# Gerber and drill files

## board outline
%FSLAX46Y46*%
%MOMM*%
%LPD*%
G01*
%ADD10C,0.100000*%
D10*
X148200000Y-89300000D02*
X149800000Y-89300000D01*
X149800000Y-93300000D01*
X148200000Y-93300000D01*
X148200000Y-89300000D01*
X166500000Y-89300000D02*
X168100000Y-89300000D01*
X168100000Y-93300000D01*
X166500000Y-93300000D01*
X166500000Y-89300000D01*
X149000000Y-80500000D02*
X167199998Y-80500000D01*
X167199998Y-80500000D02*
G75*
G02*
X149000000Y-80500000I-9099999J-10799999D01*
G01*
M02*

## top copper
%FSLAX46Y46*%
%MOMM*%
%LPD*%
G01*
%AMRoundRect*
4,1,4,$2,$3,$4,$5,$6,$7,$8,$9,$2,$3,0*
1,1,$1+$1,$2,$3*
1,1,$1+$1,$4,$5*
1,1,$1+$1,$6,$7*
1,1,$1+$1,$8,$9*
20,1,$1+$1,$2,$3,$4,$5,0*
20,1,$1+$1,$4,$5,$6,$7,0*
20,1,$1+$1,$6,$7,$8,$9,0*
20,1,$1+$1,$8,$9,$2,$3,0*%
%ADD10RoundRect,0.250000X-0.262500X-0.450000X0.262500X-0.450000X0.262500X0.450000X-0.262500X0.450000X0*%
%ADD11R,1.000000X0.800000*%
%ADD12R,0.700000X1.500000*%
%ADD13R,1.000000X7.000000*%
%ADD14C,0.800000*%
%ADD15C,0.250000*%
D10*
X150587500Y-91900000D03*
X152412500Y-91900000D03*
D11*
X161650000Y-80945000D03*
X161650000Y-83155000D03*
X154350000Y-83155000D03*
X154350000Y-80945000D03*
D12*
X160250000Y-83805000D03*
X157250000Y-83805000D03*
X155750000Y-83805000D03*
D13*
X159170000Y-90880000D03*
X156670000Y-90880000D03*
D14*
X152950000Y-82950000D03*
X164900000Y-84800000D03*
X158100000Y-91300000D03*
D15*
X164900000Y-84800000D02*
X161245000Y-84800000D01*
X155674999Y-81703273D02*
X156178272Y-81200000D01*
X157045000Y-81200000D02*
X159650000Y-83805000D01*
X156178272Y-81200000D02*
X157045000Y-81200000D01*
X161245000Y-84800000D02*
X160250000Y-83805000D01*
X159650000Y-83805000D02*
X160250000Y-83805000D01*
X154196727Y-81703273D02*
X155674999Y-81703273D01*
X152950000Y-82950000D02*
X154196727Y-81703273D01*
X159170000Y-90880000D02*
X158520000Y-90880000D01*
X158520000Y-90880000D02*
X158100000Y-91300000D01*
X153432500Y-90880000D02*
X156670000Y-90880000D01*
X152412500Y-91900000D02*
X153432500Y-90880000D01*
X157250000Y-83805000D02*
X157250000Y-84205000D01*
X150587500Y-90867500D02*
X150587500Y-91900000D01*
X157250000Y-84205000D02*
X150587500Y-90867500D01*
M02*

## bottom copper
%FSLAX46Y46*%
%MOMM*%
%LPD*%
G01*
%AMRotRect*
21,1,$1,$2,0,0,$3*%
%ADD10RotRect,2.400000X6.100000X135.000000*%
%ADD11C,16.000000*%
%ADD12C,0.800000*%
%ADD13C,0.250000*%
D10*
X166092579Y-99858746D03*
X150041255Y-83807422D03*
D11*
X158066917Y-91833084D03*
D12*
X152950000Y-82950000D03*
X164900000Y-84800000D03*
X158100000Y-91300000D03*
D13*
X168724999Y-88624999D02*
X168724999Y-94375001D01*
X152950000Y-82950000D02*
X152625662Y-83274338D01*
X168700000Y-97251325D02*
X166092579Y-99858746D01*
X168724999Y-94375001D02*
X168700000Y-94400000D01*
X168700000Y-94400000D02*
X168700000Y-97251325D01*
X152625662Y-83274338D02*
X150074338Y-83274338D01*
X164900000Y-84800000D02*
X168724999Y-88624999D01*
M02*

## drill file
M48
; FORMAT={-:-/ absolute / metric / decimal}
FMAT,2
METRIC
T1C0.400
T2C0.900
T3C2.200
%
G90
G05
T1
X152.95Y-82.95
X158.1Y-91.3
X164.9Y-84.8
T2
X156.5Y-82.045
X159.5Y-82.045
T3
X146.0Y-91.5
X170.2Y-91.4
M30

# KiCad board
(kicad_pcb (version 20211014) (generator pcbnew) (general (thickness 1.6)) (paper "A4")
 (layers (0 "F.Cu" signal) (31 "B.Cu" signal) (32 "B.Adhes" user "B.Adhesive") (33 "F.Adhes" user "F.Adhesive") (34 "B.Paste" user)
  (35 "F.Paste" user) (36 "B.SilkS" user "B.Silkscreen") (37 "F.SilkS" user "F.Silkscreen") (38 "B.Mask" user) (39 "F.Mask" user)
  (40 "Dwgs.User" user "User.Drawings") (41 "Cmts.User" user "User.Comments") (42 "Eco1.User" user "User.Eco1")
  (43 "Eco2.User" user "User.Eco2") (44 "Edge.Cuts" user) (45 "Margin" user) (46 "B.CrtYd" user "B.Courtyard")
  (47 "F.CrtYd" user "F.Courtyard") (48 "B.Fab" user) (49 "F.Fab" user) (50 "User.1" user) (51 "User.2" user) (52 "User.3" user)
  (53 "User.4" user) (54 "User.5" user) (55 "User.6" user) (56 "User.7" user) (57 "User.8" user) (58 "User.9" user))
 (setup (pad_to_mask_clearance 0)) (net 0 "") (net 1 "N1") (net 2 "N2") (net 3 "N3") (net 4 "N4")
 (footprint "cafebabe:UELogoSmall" (layer "F.Cu") (at 158.6 97)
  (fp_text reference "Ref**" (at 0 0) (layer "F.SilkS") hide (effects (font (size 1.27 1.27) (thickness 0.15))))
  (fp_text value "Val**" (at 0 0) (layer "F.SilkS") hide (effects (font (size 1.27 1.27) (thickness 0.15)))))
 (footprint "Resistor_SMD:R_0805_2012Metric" (layer "F.Cu") (at 151.5 91.9)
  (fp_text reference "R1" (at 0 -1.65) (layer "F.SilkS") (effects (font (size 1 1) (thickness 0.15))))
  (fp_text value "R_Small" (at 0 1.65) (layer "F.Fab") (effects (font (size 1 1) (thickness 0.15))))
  (pad "1" smd roundrect (at -0.9125 0) (size 1.025 1.4) (layers "F.Cu" "F.Paste" "F.Mask") (roundrect_rratio 0.243902439) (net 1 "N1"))
  (pad "2" smd roundrect (at 0.9125 0) (size 1.025 1.4) (layers "F.Cu" "F.Paste" "F.Mask") (roundrect_rratio 0.243902439) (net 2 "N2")))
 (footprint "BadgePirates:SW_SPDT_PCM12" (layer "F.Cu") (at 158 82.375 180)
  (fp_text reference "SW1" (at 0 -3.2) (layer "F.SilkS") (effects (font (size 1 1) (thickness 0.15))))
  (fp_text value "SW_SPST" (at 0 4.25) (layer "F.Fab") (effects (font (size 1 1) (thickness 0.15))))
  (pad "" smd rect locked (at -3.65 1.43 180) (size 1 0.8) (layers "F.Cu" "F.Paste" "F.Mask"))
  (pad "" np_thru_hole circle locked (at -1.5 0.33 180) (size 0.9 0.9) (drill 0.9) (layers *.Cu *.Mask))
  (pad "" smd rect locked (at -3.65 -0.78 180) (size 1 0.8) (layers "F.Cu" "F.Paste" "F.Mask"))
  (pad "" smd rect locked (at 3.65 -0.78 180) (size 1 0.8) (layers "F.Cu" "F.Paste" "F.Mask"))
  (pad "" np_thru_hole circle locked (at 1.5 0.33 180) (size 0.9 0.9) (drill 0.9) (layers *.Cu *.Mask))
  (pad "" smd rect locked (at 3.65 1.43 180) (size 1 0.8) (layers "F.Cu" "F.Paste" "F.Mask"))
  (pad "1" smd rect locked (at -2.25 -1.43 180) (size 0.7 1.5) (layers "F.Cu" "F.Paste" "F.Mask") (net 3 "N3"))
  (pad "2" smd rect locked (at 0.75 -1.43 180) (size 0.7 1.5) (layers "F.Cu" "F.Paste" "F.Mask") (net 1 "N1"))
  (pad "3" smd rect locked (at 2.25 -1.43 180) (size 0.7 1.5) (layers "F.Cu" "F.Paste" "F.Mask")))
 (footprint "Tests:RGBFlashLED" (layer "F.Cu") (at 159.17 90.88 180)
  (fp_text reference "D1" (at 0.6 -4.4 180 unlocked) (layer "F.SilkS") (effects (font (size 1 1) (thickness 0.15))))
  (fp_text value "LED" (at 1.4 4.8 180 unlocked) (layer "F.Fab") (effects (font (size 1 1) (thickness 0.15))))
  (pad "1" smd rect (at 0 0 180) (size 1 7) (layers "F.Cu" "F.Paste" "F.Mask") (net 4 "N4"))
  (pad "2" smd rect (at 2.5 0 180) (size 1 7) (layers "F.Cu" "F.Paste" "F.Mask") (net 2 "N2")))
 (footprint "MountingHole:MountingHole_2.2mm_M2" (layer "F.Cu") (at 170.2 91.4)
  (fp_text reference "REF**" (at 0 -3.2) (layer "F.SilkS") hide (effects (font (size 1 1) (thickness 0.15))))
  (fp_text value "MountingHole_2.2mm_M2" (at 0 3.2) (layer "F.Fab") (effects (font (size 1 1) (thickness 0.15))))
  (pad "" np_thru_hole circle (at 0 0) (size 2.2 2.2) (drill 2.2) (layers *.Cu *.Mask)))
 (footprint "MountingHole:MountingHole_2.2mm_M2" (layer "F.Cu") (at 146 91.5)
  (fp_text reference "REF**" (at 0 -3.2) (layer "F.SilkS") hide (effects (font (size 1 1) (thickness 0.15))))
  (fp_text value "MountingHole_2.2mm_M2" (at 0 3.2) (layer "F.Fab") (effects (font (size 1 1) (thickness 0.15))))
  (pad "" np_thru_hole circle (at 0 0) (size 2.2 2.2) (drill 2.2) (layers *.Cu *.Mask)))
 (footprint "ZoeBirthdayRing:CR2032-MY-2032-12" (layer "B.Cu") (at 158.066917 91.833084 135)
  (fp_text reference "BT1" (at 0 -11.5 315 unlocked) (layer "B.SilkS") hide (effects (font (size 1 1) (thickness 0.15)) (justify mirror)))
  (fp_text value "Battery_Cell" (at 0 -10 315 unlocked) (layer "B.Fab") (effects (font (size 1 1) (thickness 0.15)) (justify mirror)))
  (pad "1" smd rect (at -11.35 0 135) (size 2.4 6.1) (layers "B.Cu" "B.Paste" "B.Mask") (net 3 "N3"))
  (pad "1" smd rect (at 11.35 0 135) (size 2.4 6.1) (layers "B.Cu" "B.Paste" "B.Mask") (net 3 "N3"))
  (pad "2" smd circle (at 0 0 135) (size 16 16) (layers "B.Cu" "B.Paste" "B.Mask") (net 4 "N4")))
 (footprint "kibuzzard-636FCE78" (layer "B.Cu") (at 158.1 102.1 180)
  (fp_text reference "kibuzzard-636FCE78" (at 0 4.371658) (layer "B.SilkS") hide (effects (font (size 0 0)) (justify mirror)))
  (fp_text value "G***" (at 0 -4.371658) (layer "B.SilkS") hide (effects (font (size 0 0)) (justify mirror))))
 (gr_rect (start 148.2 89.3) (end 149.8 93.3) (layer "Edge.Cuts") (width 0.1) (fill none))
 (gr_rect (start 166.5 89.3) (end 168.1 93.3) (layer "Edge.Cuts") (width 0.1) (fill none))
 (gr_line (start 149 80.5) (end 167.199998 80.5) (layer "Edge.Cuts") (width 0.1))
 (gr_arc (start 167.199998 80.5) (mid 158.099999 105.422674) (end 149 80.5) (layer "Edge.Cuts") (width 0.1))
 (segment (start 164.9 84.8) (end 161.245 84.8) (width 0.25) (layer "F.Cu") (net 3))
 (segment (start 155.674999 81.703273) (end 156.178272 81.2) (width 0.25) (layer "F.Cu") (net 3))
 (segment (start 157.045 81.2) (end 159.65 83.805) (width 0.25) (layer "F.Cu") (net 3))
 (segment (start 156.178272 81.2) (end 157.045 81.2) (width 0.25) (layer "F.Cu") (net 3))
 (segment (start 161.245 84.8) (end 160.25 83.805) (width 0.25) (layer "F.Cu") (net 3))
 (segment (start 159.65 83.805) (end 160.25 83.805) (width 0.25) (layer "F.Cu") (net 3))
 (segment (start 154.196727 81.703273) (end 155.674999 81.703273) (width 0.25) (layer "F.Cu") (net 3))
 (segment (start 152.95 82.95) (end 154.196727 81.703273) (width 0.25) (layer "F.Cu") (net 3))
 (via (at 152.95 82.95) (size 0.8) (drill 0.4) (layers "F.Cu" "B.Cu") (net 3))
 (via (at 164.9 84.8) (size 0.8) (drill 0.4) (layers "F.Cu" "B.Cu") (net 3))
 (segment (start 168.724999 88.624999) (end 168.724999 94.375001) (width 0.25) (layer "B.Cu") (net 3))
 (segment (start 152.95 82.95) (end 152.625662 83.274338) (width 0.25) (layer "B.Cu") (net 3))
 (segment (start 168.7 97.251325) (end 166.092579 99.858746) (width 0.25) (layer "B.Cu") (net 3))
 (segment (start 168.724999 94.375001) (end 168.7 94.4) (width 0.25) (layer "B.Cu") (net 3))
 (segment (start 168.7 94.4) (end 168.7 97.251325) (width 0.25) (layer "B.Cu") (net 3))
 (segment (start 152.625662 83.274338) (end 150.074338 83.274338) (width 0.25) (layer "B.Cu") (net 3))
 (segment (start 164.9 84.8) (end 168.724999 88.624999) (width 0.25) (layer "B.Cu") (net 3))
 (segment (start 159.17 90.88) (end 158.52 90.88) (width 0.25) (layer "F.Cu") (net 4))
 (segment (start 158.52 90.88) (end 158.1 91.3) (width 0.25) (layer "F.Cu") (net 4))
 (via (at 158.1 91.3) (size 0.8) (drill 0.4) (layers "F.Cu" "B.Cu") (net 4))
 (segment (start 153.4325 90.88) (end 156.67 90.88) (width 0.25) (layer "F.Cu") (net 2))
 (segment (start 152.4125 91.9) (end 153.4325 90.88) (width 0.25) (layer "F.Cu") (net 2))
 (segment (start 157.25 83.805) (end 157.25 84.205) (width 0.25) (layer "F.Cu") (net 1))
 (segment (start 150.5875 90.8675) (end 150.5875 91.9) (width 0.25) (layer "F.Cu") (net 1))
 (segment (start 157.25 84.205) (end 150.5875 90.8675) (width 0.25) (layer "F.Cu") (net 1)))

